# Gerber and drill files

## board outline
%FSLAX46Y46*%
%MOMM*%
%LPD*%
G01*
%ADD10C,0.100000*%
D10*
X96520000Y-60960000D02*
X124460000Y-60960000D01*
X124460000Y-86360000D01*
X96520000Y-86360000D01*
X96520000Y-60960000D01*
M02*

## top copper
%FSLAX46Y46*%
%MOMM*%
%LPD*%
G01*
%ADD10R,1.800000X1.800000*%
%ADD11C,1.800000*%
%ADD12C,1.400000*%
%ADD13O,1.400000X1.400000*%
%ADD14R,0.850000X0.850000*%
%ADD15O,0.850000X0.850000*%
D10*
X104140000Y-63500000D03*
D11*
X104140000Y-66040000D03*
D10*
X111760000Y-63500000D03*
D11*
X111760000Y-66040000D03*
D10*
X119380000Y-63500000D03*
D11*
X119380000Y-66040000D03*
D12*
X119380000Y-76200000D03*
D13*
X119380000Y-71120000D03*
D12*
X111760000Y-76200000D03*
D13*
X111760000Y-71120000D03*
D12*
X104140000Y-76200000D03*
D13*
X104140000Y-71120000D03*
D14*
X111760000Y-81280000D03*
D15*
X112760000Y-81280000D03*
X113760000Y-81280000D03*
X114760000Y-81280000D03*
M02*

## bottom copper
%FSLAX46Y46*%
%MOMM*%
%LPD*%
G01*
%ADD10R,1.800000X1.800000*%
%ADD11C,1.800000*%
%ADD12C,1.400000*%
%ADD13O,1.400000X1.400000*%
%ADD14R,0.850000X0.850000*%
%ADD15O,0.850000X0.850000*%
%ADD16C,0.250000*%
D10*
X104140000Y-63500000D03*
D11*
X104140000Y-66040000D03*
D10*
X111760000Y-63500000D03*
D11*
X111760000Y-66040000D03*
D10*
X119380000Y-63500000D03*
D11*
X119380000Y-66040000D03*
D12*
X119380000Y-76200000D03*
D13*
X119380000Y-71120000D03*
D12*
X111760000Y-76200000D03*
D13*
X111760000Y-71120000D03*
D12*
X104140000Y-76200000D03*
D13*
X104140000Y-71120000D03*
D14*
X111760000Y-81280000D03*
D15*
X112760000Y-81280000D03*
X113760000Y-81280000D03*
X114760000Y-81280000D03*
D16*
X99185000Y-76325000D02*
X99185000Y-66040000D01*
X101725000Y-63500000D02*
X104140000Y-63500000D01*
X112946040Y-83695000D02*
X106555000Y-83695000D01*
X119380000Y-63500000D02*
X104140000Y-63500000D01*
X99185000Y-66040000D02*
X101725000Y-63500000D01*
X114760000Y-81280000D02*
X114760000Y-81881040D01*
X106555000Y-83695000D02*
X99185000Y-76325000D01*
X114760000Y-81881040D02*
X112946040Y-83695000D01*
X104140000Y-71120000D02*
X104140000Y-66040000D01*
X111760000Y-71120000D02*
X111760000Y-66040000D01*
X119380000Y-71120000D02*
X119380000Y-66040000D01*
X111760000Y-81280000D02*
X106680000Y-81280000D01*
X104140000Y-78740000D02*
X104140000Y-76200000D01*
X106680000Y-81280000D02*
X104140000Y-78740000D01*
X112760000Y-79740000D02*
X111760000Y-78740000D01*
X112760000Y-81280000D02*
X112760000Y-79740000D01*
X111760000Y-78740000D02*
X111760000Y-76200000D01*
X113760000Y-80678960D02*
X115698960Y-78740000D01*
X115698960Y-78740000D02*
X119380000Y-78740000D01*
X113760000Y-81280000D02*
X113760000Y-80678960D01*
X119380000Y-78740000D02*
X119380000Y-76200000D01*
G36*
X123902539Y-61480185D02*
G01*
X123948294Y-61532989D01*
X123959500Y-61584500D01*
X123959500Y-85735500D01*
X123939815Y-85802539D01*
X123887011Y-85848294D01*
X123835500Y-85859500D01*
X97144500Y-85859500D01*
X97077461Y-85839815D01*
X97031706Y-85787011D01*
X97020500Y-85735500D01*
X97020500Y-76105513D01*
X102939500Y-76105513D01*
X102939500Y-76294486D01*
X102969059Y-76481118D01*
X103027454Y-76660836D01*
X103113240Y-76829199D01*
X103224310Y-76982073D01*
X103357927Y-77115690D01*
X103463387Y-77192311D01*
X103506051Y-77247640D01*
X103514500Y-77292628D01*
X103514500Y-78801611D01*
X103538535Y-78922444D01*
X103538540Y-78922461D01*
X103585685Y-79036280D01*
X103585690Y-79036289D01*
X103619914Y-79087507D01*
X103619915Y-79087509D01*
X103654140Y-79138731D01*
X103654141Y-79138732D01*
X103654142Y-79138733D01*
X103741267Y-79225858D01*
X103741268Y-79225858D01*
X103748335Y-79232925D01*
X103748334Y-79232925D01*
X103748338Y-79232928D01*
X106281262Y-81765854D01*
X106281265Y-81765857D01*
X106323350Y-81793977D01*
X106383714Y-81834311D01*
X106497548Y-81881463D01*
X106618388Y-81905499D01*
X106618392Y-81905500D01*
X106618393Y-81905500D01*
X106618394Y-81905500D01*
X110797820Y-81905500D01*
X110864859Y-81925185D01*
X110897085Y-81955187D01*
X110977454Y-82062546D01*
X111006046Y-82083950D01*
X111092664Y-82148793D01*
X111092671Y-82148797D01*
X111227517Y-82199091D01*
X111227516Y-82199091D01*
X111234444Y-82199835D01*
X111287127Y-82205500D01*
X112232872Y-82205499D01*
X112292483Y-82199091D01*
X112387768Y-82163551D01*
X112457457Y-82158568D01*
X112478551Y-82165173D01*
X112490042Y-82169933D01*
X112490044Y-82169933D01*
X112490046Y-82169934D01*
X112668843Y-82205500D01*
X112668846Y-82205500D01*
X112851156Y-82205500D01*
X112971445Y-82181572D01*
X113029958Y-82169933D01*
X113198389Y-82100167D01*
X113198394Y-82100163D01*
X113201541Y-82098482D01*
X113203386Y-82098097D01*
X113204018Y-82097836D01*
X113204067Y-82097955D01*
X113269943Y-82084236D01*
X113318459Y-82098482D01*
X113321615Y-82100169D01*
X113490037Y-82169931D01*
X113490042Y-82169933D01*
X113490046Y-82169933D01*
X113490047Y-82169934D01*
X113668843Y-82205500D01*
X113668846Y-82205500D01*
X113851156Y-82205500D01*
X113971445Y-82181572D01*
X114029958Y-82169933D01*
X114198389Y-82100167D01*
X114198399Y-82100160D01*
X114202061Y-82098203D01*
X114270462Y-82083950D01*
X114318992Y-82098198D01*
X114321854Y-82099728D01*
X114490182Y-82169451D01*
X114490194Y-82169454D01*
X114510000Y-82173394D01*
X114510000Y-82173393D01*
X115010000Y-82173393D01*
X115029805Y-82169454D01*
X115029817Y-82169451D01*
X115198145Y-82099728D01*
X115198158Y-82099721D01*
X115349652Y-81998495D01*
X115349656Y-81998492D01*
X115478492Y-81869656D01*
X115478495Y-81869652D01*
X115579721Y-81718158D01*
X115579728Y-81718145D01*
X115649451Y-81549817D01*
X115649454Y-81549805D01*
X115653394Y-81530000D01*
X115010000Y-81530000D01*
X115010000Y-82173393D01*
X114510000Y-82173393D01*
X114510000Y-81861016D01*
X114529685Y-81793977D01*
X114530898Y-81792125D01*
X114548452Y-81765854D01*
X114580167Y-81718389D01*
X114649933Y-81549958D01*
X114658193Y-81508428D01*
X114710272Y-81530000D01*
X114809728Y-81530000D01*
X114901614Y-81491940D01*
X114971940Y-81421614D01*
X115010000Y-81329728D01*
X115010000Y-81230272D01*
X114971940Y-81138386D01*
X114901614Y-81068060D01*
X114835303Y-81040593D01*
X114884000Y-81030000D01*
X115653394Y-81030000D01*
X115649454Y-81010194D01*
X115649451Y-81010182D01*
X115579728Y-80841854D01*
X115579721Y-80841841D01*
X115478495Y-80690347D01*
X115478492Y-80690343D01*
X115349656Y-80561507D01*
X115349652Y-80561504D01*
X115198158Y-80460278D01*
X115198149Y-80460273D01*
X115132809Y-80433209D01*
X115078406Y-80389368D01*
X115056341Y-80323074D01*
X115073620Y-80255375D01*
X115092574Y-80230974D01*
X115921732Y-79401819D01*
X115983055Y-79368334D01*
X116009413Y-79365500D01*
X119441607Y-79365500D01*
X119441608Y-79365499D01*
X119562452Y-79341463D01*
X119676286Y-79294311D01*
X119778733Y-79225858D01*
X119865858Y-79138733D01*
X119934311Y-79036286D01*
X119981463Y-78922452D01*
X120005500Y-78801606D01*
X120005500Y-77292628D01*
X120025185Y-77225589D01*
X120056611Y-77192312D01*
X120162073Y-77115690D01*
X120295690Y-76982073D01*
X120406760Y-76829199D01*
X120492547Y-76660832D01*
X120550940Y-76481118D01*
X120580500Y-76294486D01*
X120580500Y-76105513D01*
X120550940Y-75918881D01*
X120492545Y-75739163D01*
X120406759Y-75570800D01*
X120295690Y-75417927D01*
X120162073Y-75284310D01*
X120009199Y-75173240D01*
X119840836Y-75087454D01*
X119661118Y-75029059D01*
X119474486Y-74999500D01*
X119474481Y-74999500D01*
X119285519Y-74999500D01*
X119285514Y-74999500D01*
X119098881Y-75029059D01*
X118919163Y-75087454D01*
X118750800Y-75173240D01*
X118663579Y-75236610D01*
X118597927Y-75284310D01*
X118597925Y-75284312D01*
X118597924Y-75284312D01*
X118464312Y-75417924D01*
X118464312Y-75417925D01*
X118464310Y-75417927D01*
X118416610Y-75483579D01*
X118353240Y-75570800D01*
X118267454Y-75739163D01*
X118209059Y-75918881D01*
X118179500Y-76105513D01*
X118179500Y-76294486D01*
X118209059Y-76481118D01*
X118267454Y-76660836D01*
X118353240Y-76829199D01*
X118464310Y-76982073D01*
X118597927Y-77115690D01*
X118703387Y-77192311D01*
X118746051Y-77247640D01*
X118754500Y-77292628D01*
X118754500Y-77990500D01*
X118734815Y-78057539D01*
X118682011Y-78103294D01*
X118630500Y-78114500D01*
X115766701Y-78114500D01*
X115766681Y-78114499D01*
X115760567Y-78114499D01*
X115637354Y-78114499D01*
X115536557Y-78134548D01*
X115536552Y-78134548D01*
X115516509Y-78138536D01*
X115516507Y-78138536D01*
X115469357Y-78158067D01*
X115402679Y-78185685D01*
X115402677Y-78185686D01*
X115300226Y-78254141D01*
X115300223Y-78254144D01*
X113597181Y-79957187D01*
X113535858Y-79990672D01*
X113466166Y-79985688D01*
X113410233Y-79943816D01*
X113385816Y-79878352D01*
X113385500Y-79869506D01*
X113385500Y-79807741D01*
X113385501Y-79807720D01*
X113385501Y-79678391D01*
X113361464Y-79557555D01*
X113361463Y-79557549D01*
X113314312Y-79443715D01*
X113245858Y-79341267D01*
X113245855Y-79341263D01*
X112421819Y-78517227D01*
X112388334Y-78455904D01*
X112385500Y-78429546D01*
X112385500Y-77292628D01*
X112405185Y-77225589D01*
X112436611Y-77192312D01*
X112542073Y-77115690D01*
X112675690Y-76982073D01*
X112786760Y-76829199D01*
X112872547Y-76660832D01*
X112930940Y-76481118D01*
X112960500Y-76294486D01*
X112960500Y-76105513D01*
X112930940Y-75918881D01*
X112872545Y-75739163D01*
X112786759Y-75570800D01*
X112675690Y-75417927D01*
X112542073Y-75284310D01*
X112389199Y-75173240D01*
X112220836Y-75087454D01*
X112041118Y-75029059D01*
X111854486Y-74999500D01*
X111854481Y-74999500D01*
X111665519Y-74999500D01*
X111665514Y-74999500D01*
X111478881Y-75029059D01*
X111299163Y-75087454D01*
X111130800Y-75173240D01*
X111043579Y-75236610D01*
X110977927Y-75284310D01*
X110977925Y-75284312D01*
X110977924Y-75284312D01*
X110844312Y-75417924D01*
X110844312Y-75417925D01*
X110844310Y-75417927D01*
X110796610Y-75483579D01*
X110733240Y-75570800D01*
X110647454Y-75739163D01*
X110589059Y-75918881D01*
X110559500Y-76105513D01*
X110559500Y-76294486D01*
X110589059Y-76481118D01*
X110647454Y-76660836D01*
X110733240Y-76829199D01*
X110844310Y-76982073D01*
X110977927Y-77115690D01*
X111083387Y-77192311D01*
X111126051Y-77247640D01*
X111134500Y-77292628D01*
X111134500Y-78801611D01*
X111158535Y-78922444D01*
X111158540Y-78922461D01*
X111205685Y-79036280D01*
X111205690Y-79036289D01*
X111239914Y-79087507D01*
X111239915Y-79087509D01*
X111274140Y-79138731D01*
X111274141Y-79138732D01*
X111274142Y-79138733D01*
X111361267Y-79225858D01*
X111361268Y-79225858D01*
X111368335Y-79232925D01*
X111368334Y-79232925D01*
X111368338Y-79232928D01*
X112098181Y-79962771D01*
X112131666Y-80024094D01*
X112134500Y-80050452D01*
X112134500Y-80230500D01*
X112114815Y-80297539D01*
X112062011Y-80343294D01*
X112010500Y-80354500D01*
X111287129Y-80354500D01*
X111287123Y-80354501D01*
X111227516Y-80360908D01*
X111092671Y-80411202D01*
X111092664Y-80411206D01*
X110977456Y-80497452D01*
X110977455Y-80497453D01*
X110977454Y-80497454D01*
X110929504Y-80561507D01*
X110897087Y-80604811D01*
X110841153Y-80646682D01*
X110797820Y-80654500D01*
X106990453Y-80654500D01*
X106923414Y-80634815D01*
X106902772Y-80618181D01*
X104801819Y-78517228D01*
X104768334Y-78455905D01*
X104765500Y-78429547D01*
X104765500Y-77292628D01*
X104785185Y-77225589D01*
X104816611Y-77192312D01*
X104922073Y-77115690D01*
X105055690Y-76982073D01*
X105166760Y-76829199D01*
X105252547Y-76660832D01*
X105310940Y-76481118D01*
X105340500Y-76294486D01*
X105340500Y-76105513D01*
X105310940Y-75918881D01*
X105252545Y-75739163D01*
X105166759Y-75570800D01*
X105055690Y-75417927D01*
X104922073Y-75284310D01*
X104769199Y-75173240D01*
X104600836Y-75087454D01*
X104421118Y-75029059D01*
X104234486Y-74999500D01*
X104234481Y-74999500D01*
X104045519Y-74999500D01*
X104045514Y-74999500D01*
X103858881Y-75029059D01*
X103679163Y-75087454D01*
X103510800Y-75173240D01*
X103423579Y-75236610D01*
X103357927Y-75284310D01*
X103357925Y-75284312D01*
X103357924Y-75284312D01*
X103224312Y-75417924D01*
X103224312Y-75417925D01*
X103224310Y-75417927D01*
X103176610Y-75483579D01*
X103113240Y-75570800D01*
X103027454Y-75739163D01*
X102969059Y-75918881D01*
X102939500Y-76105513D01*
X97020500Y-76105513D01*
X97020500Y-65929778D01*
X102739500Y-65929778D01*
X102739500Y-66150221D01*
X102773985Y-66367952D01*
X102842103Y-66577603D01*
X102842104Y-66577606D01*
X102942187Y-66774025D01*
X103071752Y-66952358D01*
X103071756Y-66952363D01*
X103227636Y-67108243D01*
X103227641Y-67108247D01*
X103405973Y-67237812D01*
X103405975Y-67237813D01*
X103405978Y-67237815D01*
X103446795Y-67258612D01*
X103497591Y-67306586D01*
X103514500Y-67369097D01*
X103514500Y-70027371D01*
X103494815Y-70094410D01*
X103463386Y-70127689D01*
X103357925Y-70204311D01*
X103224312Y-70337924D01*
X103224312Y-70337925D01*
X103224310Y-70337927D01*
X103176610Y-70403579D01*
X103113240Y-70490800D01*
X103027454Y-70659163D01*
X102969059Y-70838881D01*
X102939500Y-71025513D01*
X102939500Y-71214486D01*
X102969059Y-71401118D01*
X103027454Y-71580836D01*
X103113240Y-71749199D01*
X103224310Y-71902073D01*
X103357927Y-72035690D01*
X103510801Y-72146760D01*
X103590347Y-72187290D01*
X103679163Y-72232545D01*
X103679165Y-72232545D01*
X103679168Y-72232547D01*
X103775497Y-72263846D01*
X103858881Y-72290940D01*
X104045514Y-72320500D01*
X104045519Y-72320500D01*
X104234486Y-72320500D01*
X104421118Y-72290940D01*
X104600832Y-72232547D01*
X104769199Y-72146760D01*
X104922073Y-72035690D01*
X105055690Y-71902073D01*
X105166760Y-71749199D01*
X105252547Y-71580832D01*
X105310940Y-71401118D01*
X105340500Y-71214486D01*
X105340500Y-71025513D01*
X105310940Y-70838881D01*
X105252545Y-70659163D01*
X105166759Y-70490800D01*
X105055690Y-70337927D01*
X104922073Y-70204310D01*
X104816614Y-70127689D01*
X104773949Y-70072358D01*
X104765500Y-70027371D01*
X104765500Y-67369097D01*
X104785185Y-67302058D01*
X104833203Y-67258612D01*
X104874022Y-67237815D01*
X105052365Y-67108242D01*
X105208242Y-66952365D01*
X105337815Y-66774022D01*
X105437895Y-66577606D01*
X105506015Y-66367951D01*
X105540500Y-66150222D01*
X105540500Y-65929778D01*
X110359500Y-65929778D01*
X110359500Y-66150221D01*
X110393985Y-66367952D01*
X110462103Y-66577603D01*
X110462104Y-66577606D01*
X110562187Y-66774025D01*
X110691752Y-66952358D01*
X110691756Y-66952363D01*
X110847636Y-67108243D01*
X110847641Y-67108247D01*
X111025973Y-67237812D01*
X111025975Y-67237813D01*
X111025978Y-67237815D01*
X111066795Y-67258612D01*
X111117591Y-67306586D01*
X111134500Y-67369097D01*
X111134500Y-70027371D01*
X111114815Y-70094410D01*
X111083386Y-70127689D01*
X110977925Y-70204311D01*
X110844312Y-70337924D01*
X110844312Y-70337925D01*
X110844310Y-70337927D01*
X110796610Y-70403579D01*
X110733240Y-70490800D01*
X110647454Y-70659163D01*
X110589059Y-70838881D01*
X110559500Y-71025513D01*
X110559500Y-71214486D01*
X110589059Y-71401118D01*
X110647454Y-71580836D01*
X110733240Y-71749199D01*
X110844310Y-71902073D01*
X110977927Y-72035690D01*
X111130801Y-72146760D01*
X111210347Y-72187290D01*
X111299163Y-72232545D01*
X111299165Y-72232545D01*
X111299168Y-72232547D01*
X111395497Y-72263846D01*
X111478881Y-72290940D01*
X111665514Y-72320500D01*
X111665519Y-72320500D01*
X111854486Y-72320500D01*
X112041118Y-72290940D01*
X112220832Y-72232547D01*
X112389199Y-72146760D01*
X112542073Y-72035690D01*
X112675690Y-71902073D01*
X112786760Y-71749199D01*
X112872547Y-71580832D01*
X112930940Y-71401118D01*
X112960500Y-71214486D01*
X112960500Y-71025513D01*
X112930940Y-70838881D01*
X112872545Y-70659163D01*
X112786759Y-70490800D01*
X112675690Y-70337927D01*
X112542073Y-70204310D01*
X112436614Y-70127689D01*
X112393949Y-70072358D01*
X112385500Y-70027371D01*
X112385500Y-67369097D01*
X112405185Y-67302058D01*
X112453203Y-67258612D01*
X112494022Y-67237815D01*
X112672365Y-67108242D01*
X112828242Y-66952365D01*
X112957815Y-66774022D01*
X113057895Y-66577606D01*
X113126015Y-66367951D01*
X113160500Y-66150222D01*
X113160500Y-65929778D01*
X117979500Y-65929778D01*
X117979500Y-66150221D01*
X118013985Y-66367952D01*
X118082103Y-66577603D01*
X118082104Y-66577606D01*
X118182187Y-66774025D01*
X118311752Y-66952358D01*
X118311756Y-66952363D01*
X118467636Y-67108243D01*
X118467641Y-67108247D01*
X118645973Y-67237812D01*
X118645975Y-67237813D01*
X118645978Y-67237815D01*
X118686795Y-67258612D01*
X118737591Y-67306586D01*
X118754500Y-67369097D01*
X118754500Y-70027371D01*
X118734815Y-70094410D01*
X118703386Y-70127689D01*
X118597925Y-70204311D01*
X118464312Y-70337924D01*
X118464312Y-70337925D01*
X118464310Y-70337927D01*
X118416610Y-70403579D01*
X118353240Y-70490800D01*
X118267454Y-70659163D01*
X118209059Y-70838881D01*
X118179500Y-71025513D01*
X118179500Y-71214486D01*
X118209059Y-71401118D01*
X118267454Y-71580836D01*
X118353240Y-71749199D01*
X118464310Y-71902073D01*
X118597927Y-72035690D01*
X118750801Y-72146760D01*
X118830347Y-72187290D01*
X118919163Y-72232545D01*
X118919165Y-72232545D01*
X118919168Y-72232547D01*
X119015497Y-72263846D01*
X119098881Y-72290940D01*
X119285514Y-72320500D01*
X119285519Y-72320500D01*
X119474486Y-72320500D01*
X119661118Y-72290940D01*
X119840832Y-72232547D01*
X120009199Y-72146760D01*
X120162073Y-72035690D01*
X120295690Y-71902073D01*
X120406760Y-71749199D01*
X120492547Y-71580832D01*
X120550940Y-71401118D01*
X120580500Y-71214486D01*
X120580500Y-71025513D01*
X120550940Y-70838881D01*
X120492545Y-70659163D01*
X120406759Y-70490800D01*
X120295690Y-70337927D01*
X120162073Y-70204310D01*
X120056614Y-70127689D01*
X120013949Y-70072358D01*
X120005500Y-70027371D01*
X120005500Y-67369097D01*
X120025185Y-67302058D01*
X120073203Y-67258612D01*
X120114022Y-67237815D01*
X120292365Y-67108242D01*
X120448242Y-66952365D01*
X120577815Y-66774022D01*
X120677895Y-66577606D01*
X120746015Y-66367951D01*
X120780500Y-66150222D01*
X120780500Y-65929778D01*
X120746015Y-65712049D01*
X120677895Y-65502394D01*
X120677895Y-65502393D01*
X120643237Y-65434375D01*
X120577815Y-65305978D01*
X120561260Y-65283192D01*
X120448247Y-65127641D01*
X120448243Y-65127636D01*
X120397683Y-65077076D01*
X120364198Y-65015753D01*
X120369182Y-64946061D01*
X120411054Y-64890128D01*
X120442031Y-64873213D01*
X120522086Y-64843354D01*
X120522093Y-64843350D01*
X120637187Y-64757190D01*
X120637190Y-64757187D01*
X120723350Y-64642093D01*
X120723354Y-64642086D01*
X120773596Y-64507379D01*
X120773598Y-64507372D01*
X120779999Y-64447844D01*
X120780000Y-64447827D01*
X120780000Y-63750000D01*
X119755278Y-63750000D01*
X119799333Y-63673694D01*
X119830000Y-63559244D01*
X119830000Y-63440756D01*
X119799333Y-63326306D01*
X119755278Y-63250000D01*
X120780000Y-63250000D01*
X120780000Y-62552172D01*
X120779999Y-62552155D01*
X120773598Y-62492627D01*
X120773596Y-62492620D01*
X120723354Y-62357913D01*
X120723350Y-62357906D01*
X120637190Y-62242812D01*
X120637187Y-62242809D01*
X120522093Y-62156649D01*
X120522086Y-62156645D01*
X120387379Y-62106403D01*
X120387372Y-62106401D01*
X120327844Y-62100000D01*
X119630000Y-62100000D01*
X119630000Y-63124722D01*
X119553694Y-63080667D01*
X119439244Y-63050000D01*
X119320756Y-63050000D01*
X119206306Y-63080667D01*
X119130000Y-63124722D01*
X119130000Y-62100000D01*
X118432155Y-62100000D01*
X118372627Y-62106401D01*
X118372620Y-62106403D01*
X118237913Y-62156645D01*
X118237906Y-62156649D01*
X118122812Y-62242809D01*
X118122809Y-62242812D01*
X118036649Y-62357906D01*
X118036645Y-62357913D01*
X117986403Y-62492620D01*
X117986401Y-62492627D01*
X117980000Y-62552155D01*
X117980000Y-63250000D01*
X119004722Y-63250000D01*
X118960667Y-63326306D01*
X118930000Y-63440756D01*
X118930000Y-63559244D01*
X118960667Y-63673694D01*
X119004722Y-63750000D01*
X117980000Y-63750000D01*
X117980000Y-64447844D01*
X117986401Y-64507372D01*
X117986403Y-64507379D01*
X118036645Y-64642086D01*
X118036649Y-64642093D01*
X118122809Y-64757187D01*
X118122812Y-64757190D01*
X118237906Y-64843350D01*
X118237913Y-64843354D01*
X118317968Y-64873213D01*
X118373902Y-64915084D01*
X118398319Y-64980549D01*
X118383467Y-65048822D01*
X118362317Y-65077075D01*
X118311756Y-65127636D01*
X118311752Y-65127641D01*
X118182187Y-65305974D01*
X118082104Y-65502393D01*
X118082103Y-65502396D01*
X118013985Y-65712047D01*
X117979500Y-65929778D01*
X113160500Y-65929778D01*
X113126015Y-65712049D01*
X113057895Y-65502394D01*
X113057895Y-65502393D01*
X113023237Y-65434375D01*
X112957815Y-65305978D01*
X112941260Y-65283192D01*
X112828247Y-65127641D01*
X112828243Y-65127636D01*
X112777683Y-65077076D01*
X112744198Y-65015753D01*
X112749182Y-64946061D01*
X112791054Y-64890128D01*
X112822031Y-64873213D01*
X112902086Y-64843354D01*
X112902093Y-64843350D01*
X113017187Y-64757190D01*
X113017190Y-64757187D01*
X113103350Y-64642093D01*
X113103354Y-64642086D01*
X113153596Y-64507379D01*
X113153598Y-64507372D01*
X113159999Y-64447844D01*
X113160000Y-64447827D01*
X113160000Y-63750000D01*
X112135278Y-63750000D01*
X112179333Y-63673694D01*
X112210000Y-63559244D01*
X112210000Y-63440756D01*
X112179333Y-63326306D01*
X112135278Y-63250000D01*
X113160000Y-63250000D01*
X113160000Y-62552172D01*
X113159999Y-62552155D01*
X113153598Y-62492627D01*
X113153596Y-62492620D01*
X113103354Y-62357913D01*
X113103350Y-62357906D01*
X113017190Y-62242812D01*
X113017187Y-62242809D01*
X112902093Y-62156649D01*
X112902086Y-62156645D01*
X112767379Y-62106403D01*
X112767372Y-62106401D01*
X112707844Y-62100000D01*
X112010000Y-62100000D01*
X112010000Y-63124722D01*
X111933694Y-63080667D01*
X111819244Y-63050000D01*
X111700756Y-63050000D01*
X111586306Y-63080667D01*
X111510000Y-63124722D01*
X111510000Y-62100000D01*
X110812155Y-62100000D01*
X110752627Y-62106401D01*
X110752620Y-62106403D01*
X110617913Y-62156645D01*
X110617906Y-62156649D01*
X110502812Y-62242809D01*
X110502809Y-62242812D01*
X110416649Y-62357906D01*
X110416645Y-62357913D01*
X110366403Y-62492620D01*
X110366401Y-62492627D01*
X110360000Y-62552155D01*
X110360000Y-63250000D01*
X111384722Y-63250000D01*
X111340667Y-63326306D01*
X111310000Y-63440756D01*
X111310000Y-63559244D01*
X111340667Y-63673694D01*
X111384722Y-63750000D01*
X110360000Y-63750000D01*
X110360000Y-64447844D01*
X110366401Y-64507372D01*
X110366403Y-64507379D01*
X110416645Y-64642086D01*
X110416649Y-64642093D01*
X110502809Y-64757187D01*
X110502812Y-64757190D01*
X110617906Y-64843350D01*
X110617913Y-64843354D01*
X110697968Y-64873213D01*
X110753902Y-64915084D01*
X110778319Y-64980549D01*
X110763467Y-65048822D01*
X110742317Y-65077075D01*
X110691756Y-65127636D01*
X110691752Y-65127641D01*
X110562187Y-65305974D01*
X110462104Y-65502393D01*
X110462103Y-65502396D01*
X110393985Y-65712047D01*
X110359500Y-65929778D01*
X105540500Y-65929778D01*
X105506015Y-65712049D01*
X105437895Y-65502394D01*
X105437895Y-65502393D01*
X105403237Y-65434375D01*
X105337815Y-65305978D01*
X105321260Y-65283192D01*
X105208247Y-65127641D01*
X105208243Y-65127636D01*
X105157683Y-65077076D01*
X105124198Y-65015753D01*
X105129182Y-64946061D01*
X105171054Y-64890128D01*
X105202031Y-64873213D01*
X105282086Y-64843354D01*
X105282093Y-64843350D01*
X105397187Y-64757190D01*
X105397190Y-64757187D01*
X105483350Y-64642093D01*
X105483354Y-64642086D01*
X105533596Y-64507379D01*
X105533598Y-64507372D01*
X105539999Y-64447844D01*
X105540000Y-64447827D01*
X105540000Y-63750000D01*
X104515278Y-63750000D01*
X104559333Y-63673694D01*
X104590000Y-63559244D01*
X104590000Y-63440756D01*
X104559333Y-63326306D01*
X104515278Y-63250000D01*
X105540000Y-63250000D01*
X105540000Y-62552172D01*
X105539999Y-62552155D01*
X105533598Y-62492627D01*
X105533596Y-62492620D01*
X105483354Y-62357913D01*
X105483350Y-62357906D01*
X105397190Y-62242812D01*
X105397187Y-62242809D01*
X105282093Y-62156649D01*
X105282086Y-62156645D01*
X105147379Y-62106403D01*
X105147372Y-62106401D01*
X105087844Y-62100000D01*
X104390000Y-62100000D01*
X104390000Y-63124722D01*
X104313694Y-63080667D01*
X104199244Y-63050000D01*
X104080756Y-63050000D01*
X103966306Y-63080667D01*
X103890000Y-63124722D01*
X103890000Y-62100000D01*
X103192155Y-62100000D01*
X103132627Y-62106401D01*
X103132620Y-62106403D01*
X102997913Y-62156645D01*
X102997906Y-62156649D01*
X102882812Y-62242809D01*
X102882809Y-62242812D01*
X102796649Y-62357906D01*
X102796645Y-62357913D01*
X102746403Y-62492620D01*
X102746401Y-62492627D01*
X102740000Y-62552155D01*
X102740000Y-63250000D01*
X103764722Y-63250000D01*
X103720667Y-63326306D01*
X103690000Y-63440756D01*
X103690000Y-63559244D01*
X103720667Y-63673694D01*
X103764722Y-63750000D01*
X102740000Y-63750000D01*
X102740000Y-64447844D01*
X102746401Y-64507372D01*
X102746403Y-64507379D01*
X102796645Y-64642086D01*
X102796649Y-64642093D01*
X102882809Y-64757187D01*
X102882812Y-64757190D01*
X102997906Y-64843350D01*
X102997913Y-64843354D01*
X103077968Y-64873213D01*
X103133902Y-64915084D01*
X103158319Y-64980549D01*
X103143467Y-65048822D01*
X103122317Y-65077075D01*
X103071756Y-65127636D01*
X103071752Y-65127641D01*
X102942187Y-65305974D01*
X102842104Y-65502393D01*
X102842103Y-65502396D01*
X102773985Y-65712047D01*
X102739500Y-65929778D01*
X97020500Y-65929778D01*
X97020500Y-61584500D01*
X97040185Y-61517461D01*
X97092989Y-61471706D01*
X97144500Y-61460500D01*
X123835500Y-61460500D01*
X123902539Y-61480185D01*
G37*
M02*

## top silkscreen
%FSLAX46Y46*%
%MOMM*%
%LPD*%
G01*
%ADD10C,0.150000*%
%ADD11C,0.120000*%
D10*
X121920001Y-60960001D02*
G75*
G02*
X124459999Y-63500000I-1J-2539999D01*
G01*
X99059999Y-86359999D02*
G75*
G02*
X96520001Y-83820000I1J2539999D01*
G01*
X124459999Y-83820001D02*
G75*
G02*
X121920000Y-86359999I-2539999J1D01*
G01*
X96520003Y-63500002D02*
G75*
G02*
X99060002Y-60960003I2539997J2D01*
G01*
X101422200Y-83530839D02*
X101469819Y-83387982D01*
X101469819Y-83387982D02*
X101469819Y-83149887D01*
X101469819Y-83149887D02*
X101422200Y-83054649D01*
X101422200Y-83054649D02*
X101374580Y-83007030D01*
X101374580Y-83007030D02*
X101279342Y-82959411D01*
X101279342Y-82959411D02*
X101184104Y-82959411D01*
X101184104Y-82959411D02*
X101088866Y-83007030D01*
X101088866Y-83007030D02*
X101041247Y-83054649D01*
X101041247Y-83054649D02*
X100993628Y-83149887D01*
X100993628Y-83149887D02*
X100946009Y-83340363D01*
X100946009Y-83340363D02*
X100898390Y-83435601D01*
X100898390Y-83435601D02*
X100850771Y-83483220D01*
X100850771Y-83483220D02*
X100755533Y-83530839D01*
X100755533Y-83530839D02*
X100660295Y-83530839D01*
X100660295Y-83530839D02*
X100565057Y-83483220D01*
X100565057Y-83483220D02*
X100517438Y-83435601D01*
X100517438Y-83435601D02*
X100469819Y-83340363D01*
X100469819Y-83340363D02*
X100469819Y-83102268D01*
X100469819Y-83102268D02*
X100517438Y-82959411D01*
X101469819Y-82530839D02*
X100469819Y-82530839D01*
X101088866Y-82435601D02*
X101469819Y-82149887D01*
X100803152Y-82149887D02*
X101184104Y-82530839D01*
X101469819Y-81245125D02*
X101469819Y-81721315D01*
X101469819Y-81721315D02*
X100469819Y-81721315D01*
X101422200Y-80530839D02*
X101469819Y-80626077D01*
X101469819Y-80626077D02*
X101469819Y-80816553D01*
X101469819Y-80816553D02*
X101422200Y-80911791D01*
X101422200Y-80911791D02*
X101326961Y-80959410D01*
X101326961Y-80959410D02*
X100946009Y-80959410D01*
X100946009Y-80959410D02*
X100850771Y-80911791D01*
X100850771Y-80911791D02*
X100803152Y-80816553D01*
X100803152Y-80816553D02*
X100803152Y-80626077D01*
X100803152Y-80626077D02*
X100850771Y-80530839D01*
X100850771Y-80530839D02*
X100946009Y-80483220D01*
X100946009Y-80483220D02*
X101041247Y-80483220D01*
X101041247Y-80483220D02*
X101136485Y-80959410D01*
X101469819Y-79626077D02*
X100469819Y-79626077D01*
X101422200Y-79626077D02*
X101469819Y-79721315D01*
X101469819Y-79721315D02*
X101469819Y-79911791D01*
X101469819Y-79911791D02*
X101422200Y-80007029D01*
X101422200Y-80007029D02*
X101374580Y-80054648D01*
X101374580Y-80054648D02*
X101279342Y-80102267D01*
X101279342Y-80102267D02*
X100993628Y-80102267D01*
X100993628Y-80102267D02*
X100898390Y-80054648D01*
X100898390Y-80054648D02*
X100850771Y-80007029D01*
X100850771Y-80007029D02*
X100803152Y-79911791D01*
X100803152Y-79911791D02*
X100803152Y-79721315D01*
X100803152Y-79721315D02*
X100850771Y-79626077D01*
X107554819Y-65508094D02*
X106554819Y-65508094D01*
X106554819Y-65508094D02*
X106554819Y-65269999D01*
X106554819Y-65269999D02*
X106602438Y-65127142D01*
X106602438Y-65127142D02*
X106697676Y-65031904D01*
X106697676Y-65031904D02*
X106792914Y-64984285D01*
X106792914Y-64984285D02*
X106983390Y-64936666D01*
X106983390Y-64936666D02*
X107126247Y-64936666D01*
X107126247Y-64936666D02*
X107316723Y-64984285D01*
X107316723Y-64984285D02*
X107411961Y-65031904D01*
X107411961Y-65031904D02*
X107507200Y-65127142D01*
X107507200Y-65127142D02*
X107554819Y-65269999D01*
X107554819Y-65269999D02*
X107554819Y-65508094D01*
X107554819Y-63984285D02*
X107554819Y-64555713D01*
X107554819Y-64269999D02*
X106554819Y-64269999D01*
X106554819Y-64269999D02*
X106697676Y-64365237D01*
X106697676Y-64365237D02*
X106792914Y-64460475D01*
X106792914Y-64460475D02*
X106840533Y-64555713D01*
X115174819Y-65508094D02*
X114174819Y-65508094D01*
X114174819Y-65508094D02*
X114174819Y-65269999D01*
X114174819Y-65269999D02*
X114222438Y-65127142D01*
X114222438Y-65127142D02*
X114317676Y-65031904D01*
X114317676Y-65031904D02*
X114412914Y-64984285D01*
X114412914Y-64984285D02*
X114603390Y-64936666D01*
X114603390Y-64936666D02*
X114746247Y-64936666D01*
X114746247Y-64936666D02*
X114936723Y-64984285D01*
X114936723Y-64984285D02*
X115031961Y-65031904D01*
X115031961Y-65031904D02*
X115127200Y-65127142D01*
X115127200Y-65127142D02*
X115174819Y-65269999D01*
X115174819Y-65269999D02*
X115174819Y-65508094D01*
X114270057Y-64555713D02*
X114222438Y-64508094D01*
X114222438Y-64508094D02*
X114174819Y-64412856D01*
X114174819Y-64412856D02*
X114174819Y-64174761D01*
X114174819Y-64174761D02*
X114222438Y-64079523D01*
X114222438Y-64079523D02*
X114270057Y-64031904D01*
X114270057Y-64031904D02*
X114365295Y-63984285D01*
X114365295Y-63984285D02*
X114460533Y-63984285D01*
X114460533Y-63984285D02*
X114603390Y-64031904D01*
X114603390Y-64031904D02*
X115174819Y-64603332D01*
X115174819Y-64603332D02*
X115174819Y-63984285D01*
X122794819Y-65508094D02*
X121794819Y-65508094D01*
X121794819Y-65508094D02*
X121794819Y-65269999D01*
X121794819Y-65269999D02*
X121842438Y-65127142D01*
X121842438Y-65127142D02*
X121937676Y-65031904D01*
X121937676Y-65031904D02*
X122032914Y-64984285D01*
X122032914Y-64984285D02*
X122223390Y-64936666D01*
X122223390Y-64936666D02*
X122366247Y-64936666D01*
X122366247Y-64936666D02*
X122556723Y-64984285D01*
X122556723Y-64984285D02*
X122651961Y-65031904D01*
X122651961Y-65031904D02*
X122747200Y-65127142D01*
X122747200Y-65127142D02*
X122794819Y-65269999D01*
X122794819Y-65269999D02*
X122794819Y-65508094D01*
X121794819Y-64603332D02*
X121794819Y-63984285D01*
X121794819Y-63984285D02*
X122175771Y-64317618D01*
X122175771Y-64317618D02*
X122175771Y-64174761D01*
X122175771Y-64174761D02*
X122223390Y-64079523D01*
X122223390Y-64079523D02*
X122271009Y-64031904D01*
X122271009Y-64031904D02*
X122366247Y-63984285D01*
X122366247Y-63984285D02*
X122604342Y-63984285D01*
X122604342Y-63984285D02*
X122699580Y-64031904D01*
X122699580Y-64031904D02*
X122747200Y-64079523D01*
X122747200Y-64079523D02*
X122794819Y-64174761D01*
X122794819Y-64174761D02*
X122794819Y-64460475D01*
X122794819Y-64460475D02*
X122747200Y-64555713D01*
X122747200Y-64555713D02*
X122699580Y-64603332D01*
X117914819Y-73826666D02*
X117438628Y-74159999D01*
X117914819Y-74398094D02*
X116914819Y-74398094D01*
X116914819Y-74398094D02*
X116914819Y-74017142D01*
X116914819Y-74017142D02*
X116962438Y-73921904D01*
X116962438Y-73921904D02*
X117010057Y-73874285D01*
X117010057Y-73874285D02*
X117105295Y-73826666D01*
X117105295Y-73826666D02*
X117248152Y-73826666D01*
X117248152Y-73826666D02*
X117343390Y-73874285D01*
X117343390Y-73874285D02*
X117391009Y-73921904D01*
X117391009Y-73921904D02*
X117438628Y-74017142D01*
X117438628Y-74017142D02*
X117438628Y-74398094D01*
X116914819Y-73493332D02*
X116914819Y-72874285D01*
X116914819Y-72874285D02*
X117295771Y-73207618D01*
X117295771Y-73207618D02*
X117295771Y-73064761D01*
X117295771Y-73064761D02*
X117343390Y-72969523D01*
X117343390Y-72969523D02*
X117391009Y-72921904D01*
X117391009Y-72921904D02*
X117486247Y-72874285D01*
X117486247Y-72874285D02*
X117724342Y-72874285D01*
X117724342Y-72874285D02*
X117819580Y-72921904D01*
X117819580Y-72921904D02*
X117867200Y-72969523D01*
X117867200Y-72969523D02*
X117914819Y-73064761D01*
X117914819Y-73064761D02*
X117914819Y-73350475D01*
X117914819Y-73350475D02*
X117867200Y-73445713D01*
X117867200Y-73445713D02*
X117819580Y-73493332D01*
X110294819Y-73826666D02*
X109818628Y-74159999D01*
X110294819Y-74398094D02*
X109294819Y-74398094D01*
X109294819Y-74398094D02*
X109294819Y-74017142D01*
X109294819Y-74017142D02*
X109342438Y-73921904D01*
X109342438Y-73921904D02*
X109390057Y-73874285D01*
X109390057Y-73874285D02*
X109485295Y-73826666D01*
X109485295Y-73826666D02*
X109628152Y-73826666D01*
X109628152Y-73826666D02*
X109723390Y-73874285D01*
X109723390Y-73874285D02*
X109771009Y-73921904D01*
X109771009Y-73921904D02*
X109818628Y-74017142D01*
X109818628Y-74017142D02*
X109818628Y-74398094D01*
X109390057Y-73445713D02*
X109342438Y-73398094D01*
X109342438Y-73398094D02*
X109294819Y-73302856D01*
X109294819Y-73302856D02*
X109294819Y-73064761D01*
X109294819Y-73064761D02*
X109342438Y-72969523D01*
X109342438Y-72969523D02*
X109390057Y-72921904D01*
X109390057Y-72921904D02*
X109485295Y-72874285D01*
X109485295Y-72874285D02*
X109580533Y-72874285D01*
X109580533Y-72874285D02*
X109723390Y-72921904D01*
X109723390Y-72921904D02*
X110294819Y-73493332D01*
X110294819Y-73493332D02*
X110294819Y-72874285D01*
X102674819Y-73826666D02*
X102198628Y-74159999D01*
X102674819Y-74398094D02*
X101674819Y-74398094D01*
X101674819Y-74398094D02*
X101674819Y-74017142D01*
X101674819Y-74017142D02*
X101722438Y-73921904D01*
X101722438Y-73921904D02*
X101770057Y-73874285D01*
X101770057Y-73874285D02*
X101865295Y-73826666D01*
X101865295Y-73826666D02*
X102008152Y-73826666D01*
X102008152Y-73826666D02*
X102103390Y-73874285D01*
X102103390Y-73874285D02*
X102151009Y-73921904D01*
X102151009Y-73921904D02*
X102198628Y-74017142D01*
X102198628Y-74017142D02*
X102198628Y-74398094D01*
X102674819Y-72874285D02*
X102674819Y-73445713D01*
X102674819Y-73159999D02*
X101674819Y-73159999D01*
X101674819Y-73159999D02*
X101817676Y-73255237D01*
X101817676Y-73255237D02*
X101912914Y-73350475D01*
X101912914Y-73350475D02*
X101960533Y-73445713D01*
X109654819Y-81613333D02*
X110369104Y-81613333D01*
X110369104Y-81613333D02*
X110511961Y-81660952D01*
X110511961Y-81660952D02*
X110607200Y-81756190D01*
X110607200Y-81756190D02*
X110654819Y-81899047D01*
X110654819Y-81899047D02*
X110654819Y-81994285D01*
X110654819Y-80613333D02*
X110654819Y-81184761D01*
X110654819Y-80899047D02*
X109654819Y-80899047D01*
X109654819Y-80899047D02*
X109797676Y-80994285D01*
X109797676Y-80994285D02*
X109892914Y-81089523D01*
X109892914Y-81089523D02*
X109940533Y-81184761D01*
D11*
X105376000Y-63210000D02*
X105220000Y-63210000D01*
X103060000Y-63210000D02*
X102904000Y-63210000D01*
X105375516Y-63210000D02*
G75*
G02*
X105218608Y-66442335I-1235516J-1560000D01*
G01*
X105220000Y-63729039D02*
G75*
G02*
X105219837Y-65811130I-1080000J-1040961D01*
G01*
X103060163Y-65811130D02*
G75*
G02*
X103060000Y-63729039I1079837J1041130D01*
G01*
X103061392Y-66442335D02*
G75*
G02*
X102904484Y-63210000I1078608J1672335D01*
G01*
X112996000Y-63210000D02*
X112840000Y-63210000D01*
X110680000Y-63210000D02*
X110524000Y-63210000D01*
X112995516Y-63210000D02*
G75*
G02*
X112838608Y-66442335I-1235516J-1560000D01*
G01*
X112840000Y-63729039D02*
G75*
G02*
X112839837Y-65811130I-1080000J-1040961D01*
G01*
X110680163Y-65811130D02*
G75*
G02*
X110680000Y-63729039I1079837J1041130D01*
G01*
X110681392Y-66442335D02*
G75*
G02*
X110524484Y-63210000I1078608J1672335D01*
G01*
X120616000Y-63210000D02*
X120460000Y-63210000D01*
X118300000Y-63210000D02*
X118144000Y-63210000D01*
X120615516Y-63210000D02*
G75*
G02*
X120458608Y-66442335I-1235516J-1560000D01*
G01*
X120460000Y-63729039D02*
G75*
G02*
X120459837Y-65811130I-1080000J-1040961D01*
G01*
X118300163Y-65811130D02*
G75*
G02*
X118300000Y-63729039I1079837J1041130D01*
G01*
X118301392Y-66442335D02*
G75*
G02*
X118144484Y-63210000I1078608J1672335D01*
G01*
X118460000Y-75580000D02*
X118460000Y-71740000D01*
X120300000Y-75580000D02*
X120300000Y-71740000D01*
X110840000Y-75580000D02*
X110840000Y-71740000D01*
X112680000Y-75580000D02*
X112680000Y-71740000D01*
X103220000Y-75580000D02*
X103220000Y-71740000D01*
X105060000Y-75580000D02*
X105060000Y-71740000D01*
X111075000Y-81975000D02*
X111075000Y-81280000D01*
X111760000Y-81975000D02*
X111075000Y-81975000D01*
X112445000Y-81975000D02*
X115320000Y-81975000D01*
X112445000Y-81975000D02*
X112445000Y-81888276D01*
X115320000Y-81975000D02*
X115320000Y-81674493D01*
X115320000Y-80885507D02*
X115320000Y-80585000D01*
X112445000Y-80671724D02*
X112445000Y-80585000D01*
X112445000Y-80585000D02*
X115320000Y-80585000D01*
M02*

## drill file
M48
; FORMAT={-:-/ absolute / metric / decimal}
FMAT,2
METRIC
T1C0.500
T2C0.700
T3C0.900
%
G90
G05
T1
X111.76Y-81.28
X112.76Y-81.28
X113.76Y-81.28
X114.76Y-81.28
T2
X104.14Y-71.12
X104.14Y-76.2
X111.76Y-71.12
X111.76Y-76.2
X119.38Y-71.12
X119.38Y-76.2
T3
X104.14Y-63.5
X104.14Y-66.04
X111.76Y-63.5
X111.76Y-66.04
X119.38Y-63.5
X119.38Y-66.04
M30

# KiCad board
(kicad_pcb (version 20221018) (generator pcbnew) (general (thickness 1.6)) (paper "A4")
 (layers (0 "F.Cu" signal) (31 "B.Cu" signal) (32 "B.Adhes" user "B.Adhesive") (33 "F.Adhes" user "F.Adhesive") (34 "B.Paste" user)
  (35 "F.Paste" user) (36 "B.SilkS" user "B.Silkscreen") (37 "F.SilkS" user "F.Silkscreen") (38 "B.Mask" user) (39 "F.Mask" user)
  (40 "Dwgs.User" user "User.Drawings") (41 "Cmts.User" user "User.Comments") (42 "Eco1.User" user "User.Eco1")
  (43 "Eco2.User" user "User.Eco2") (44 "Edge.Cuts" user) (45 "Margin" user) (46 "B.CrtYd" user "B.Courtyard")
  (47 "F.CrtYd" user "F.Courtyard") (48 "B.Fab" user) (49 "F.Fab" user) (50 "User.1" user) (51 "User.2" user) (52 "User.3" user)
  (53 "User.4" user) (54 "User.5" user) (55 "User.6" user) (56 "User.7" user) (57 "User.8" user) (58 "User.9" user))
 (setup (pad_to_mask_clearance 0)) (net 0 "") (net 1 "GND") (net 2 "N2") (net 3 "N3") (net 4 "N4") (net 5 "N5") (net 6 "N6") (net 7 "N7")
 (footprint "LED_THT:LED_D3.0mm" (layer "F.Cu") (at 104.14 63.5 -90)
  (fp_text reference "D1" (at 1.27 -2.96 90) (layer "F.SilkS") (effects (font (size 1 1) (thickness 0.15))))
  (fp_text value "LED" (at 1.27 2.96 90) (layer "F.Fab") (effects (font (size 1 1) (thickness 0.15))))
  (fp_line (start -0.29 -1.236) (end -0.29 -1.08) (stroke (width 0.12) (type solid)) (layer "F.SilkS"))
  (fp_line (start -0.29 1.08) (end -0.29 1.236) (stroke (width 0.12) (type solid)) (layer "F.SilkS"))
  (fp_arc (start -0.29 -1.235516) (mid 1.366487 -1.987659) (end 2.942335 -1.078608) (stroke (width 0.12) (type solid)) (layer "F.SilkS"))
  (fp_arc (start 0.229039 -1.08) (mid 1.270117 -1.5) (end 2.31113 -1.079837) (stroke (width 0.12) (type solid)) (layer "F.SilkS"))
  (fp_arc (start 2.31113 1.079837) (mid 1.270117 1.5) (end 0.229039 1.08) (stroke (width 0.12) (type solid)) (layer "F.SilkS"))
  (fp_arc (start 2.942335 1.078608) (mid 1.366487 1.987659) (end -0.29 1.235516) (stroke (width 0.12) (type solid)) (layer "F.SilkS"))
  (pad "1" thru_hole rect (at 0 0 270) (size 1.8 1.8) (drill 0.9) (layers "*.Cu" "*.Mask") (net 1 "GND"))
  (pad "2" thru_hole circle (at 2.54 0 270) (size 1.8 1.8) (drill 0.9) (layers "*.Cu" "*.Mask") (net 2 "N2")))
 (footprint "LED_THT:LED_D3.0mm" (layer "F.Cu") (at 111.76 63.5 -90)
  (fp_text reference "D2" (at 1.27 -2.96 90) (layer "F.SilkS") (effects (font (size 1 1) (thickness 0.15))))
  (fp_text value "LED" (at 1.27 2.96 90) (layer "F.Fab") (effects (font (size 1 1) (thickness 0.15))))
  (fp_line (start -0.29 -1.236) (end -0.29 -1.08) (stroke (width 0.12) (type solid)) (layer "F.SilkS"))
  (fp_line (start -0.29 1.08) (end -0.29 1.236) (stroke (width 0.12) (type solid)) (layer "F.SilkS"))
  (fp_arc (start -0.29 -1.235516) (mid 1.366487 -1.987659) (end 2.942335 -1.078608) (stroke (width 0.12) (type solid)) (layer "F.SilkS"))
  (fp_arc (start 0.229039 -1.08) (mid 1.270117 -1.5) (end 2.31113 -1.079837) (stroke (width 0.12) (type solid)) (layer "F.SilkS"))
  (fp_arc (start 2.31113 1.079837) (mid 1.270117 1.5) (end 0.229039 1.08) (stroke (width 0.12) (type solid)) (layer "F.SilkS"))
  (fp_arc (start 2.942335 1.078608) (mid 1.366487 1.987659) (end -0.29 1.235516) (stroke (width 0.12) (type solid)) (layer "F.SilkS"))
  (pad "1" thru_hole rect (at 0 0 270) (size 1.8 1.8) (drill 0.9) (layers "*.Cu" "*.Mask") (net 1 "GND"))
  (pad "2" thru_hole circle (at 2.54 0 270) (size 1.8 1.8) (drill 0.9) (layers "*.Cu" "*.Mask") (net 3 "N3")))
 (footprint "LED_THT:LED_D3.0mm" (layer "F.Cu") (at 119.38 63.5 -90)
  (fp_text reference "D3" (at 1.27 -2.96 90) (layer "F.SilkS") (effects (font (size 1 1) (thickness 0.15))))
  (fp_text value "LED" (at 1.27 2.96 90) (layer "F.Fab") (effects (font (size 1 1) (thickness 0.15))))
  (fp_line (start -0.29 -1.236) (end -0.29 -1.08) (stroke (width 0.12) (type solid)) (layer "F.SilkS"))
  (fp_line (start -0.29 1.08) (end -0.29 1.236) (stroke (width 0.12) (type solid)) (layer "F.SilkS"))
  (fp_arc (start -0.29 -1.235516) (mid 1.366487 -1.987659) (end 2.942335 -1.078608) (stroke (width 0.12) (type solid)) (layer "F.SilkS"))
  (fp_arc (start 0.229039 -1.08) (mid 1.270117 -1.5) (end 2.31113 -1.079837) (stroke (width 0.12) (type solid)) (layer "F.SilkS"))
  (fp_arc (start 2.31113 1.079837) (mid 1.270117 1.5) (end 0.229039 1.08) (stroke (width 0.12) (type solid)) (layer "F.SilkS"))
  (fp_arc (start 2.942335 1.078608) (mid 1.366487 1.987659) (end -0.29 1.235516) (stroke (width 0.12) (type solid)) (layer "F.SilkS"))
  (pad "1" thru_hole rect (at 0 0 270) (size 1.8 1.8) (drill 0.9) (layers "*.Cu" "*.Mask") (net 1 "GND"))
  (pad "2" thru_hole circle (at 2.54 0 270) (size 1.8 1.8) (drill 0.9) (layers "*.Cu" "*.Mask") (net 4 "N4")))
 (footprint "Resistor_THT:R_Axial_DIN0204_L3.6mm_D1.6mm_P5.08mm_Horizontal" (layer "F.Cu") (at 119.38 76.2 90)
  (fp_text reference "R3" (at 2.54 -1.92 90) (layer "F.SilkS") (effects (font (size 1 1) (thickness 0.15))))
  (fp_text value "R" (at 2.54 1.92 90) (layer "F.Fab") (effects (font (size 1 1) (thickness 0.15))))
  (fp_line (start 0.62 -0.92) (end 4.46 -0.92) (stroke (width 0.12) (type solid)) (layer "F.SilkS"))
  (fp_line (start 0.62 0.92) (end 4.46 0.92) (stroke (width 0.12) (type solid)) (layer "F.SilkS"))
  (pad "1" thru_hole circle (at 0 0 90) (size 1.4 1.4) (drill 0.7) (layers "*.Cu" "*.Mask") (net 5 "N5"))
  (pad "2" thru_hole oval (at 5.08 0 90) (size 1.4 1.4) (drill 0.7) (layers "*.Cu" "*.Mask") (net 4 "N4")))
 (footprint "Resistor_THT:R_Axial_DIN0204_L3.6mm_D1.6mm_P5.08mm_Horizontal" (layer "F.Cu") (at 111.76 76.2 90)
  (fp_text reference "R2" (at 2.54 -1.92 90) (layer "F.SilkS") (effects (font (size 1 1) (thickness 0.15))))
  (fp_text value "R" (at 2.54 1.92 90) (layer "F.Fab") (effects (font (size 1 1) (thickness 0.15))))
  (fp_line (start 0.62 -0.92) (end 4.46 -0.92) (stroke (width 0.12) (type solid)) (layer "F.SilkS"))
  (fp_line (start 0.62 0.92) (end 4.46 0.92) (stroke (width 0.12) (type solid)) (layer "F.SilkS"))
  (pad "1" thru_hole circle (at 0 0 90) (size 1.4 1.4) (drill 0.7) (layers "*.Cu" "*.Mask") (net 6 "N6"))
  (pad "2" thru_hole oval (at 5.08 0 90) (size 1.4 1.4) (drill 0.7) (layers "*.Cu" "*.Mask") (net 3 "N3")))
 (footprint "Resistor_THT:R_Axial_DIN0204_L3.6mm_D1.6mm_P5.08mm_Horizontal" (layer "F.Cu") (at 104.14 76.2 90)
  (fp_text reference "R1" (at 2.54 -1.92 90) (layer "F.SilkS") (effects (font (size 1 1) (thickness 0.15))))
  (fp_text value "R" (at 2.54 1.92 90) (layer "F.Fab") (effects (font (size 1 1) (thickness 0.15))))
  (fp_line (start 0.62 -0.92) (end 4.46 -0.92) (stroke (width 0.12) (type solid)) (layer "F.SilkS"))
  (fp_line (start 0.62 0.92) (end 4.46 0.92) (stroke (width 0.12) (type solid)) (layer "F.SilkS"))
  (pad "1" thru_hole circle (at 0 0 90) (size 1.4 1.4) (drill 0.7) (layers "*.Cu" "*.Mask") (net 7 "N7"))
  (pad "2" thru_hole oval (at 5.08 0 90) (size 1.4 1.4) (drill 0.7) (layers "*.Cu" "*.Mask") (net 2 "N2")))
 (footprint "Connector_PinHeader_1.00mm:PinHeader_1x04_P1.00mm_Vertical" (layer "F.Cu") (at 111.76 81.28 90)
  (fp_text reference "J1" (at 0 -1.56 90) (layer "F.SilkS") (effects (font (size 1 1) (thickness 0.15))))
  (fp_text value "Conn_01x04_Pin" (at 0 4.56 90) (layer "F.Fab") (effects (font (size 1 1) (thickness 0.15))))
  (fp_line (start -0.695 -0.685) (end 0 -0.685) (stroke (width 0.12) (type solid)) (layer "F.SilkS"))
  (fp_line (start -0.695 0) (end -0.695 -0.685) (stroke (width 0.12) (type solid)) (layer "F.SilkS"))
  (fp_line (start -0.695 0.685) (end -0.695 3.56) (stroke (width 0.12) (type solid)) (layer "F.SilkS"))
  (fp_line (start -0.695 0.685) (end -0.608276 0.685) (stroke (width 0.12) (type solid)) (layer "F.SilkS"))
  (fp_line (start -0.695 3.56) (end -0.394493 3.56) (stroke (width 0.12) (type solid)) (layer "F.SilkS"))
  (fp_line (start 0.394493 3.56) (end 0.695 3.56) (stroke (width 0.12) (type solid)) (layer "F.SilkS"))
  (fp_line (start 0.608276 0.685) (end 0.695 0.685) (stroke (width 0.12) (type solid)) (layer "F.SilkS"))
  (fp_line (start 0.695 0.685) (end 0.695 3.56) (stroke (width 0.12) (type solid)) (layer "F.SilkS"))
  (pad "1" thru_hole rect (at 0 0 90) (size 0.85 0.85) (drill 0.5) (layers "*.Cu" "*.Mask") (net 7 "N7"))
  (pad "2" thru_hole oval (at 0 1 90) (size 0.85 0.85) (drill 0.5) (layers "*.Cu" "*.Mask") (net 6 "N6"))
  (pad "3" thru_hole oval (at 0 2 90) (size 0.85 0.85) (drill 0.5) (layers "*.Cu" "*.Mask") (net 5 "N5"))
  (pad "4" thru_hole oval (at 0 3 90) (size 0.85 0.85) (drill 0.5) (layers "*.Cu" "*.Mask") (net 1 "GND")))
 (gr_arc (start 121.920001 60.960001) (mid 123.716052 61.703949) (end 124.46 63.5) (stroke (width 0.15) (type default)) (layer "F.SilkS"))
 (gr_arc (start 99.059999 86.359999) (mid 97.263948 85.616051) (end 96.52 83.82) (stroke (width 0.15) (type default)) (layer "F.SilkS"))
 (gr_arc (start 124.459999 83.820001) (mid 123.716051 85.616052) (end 121.92 86.36) (stroke (width 0.15) (type default)) (layer "F.SilkS"))
 (gr_arc (start 96.520003 63.500002) (mid 97.263951 61.703951) (end 99.060002 60.960003) (stroke (width 0.15) (type default))
  (layer "F.SilkS"))
 (gr_poly
  (pts (xy 96.52 60.96) (xy 124.46 60.96) (xy 124.46 86.36) (xy 96.52 86.36)) (stroke (width 0.1) (type solid)) (fill none)
  (layer "Edge.Cuts"))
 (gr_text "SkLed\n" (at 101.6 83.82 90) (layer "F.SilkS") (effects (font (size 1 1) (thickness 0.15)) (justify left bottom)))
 (segment (start 99.185 76.325) (end 99.185 66.04) (width 0.25) (layer "B.Cu") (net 1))
 (segment (start 101.725 63.5) (end 104.14 63.5) (width 0.25) (layer "B.Cu") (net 1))
 (segment (start 112.94604 83.695) (end 106.555 83.695) (width 0.25) (layer "B.Cu") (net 1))
 (segment (start 119.38 63.5) (end 104.14 63.5) (width 0.25) (layer "B.Cu") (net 1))
 (segment (start 99.185 66.04) (end 101.725 63.5) (width 0.25) (layer "B.Cu") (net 1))
 (segment (start 114.76 81.28) (end 114.76 81.88104) (width 0.25) (layer "B.Cu") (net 1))
 (segment (start 106.555 83.695) (end 99.185 76.325) (width 0.25) (layer "B.Cu") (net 1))
 (segment (start 114.76 81.88104) (end 112.94604 83.695) (width 0.25) (layer "B.Cu") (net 1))
 (segment (start 104.14 71.12) (end 104.14 66.04) (width 0.25) (layer "B.Cu") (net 2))
 (segment (start 111.76 71.12) (end 111.76 66.04) (width 0.25) (layer "B.Cu") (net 3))
 (segment (start 119.38 71.12) (end 119.38 66.04) (width 0.25) (layer "B.Cu") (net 4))
 (segment (start 111.76 81.28) (end 106.68 81.28) (width 0.25) (layer "B.Cu") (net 7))
 (segment (start 104.14 78.74) (end 104.14 76.2) (width 0.25) (layer "B.Cu") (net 7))
 (segment (start 106.68 81.28) (end 104.14 78.74) (width 0.25) (layer "B.Cu") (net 7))
 (segment (start 112.76 79.74) (end 111.76 78.74) (width 0.25) (layer "B.Cu") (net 6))
 (segment (start 112.76 81.28) (end 112.76 79.74) (width 0.25) (layer "B.Cu") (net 6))
 (segment (start 111.76 78.74) (end 111.76 76.2) (width 0.25) (layer "B.Cu") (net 6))
 (segment (start 113.76 80.67896) (end 115.69896 78.74) (width 0.25) (layer "B.Cu") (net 5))
 (segment (start 115.69896 78.74) (end 119.38 78.74) (width 0.25) (layer "B.Cu") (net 5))
 (segment (start 113.76 81.28) (end 113.76 80.67896) (width 0.25) (layer "B.Cu") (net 5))
 (segment (start 119.38 78.74) (end 119.38 76.2) (width 0.25) (layer "B.Cu") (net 5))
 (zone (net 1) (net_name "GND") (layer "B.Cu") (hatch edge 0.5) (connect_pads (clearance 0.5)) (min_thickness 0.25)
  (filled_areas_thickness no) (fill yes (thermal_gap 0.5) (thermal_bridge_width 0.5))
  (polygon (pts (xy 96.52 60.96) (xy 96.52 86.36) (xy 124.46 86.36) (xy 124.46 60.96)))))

